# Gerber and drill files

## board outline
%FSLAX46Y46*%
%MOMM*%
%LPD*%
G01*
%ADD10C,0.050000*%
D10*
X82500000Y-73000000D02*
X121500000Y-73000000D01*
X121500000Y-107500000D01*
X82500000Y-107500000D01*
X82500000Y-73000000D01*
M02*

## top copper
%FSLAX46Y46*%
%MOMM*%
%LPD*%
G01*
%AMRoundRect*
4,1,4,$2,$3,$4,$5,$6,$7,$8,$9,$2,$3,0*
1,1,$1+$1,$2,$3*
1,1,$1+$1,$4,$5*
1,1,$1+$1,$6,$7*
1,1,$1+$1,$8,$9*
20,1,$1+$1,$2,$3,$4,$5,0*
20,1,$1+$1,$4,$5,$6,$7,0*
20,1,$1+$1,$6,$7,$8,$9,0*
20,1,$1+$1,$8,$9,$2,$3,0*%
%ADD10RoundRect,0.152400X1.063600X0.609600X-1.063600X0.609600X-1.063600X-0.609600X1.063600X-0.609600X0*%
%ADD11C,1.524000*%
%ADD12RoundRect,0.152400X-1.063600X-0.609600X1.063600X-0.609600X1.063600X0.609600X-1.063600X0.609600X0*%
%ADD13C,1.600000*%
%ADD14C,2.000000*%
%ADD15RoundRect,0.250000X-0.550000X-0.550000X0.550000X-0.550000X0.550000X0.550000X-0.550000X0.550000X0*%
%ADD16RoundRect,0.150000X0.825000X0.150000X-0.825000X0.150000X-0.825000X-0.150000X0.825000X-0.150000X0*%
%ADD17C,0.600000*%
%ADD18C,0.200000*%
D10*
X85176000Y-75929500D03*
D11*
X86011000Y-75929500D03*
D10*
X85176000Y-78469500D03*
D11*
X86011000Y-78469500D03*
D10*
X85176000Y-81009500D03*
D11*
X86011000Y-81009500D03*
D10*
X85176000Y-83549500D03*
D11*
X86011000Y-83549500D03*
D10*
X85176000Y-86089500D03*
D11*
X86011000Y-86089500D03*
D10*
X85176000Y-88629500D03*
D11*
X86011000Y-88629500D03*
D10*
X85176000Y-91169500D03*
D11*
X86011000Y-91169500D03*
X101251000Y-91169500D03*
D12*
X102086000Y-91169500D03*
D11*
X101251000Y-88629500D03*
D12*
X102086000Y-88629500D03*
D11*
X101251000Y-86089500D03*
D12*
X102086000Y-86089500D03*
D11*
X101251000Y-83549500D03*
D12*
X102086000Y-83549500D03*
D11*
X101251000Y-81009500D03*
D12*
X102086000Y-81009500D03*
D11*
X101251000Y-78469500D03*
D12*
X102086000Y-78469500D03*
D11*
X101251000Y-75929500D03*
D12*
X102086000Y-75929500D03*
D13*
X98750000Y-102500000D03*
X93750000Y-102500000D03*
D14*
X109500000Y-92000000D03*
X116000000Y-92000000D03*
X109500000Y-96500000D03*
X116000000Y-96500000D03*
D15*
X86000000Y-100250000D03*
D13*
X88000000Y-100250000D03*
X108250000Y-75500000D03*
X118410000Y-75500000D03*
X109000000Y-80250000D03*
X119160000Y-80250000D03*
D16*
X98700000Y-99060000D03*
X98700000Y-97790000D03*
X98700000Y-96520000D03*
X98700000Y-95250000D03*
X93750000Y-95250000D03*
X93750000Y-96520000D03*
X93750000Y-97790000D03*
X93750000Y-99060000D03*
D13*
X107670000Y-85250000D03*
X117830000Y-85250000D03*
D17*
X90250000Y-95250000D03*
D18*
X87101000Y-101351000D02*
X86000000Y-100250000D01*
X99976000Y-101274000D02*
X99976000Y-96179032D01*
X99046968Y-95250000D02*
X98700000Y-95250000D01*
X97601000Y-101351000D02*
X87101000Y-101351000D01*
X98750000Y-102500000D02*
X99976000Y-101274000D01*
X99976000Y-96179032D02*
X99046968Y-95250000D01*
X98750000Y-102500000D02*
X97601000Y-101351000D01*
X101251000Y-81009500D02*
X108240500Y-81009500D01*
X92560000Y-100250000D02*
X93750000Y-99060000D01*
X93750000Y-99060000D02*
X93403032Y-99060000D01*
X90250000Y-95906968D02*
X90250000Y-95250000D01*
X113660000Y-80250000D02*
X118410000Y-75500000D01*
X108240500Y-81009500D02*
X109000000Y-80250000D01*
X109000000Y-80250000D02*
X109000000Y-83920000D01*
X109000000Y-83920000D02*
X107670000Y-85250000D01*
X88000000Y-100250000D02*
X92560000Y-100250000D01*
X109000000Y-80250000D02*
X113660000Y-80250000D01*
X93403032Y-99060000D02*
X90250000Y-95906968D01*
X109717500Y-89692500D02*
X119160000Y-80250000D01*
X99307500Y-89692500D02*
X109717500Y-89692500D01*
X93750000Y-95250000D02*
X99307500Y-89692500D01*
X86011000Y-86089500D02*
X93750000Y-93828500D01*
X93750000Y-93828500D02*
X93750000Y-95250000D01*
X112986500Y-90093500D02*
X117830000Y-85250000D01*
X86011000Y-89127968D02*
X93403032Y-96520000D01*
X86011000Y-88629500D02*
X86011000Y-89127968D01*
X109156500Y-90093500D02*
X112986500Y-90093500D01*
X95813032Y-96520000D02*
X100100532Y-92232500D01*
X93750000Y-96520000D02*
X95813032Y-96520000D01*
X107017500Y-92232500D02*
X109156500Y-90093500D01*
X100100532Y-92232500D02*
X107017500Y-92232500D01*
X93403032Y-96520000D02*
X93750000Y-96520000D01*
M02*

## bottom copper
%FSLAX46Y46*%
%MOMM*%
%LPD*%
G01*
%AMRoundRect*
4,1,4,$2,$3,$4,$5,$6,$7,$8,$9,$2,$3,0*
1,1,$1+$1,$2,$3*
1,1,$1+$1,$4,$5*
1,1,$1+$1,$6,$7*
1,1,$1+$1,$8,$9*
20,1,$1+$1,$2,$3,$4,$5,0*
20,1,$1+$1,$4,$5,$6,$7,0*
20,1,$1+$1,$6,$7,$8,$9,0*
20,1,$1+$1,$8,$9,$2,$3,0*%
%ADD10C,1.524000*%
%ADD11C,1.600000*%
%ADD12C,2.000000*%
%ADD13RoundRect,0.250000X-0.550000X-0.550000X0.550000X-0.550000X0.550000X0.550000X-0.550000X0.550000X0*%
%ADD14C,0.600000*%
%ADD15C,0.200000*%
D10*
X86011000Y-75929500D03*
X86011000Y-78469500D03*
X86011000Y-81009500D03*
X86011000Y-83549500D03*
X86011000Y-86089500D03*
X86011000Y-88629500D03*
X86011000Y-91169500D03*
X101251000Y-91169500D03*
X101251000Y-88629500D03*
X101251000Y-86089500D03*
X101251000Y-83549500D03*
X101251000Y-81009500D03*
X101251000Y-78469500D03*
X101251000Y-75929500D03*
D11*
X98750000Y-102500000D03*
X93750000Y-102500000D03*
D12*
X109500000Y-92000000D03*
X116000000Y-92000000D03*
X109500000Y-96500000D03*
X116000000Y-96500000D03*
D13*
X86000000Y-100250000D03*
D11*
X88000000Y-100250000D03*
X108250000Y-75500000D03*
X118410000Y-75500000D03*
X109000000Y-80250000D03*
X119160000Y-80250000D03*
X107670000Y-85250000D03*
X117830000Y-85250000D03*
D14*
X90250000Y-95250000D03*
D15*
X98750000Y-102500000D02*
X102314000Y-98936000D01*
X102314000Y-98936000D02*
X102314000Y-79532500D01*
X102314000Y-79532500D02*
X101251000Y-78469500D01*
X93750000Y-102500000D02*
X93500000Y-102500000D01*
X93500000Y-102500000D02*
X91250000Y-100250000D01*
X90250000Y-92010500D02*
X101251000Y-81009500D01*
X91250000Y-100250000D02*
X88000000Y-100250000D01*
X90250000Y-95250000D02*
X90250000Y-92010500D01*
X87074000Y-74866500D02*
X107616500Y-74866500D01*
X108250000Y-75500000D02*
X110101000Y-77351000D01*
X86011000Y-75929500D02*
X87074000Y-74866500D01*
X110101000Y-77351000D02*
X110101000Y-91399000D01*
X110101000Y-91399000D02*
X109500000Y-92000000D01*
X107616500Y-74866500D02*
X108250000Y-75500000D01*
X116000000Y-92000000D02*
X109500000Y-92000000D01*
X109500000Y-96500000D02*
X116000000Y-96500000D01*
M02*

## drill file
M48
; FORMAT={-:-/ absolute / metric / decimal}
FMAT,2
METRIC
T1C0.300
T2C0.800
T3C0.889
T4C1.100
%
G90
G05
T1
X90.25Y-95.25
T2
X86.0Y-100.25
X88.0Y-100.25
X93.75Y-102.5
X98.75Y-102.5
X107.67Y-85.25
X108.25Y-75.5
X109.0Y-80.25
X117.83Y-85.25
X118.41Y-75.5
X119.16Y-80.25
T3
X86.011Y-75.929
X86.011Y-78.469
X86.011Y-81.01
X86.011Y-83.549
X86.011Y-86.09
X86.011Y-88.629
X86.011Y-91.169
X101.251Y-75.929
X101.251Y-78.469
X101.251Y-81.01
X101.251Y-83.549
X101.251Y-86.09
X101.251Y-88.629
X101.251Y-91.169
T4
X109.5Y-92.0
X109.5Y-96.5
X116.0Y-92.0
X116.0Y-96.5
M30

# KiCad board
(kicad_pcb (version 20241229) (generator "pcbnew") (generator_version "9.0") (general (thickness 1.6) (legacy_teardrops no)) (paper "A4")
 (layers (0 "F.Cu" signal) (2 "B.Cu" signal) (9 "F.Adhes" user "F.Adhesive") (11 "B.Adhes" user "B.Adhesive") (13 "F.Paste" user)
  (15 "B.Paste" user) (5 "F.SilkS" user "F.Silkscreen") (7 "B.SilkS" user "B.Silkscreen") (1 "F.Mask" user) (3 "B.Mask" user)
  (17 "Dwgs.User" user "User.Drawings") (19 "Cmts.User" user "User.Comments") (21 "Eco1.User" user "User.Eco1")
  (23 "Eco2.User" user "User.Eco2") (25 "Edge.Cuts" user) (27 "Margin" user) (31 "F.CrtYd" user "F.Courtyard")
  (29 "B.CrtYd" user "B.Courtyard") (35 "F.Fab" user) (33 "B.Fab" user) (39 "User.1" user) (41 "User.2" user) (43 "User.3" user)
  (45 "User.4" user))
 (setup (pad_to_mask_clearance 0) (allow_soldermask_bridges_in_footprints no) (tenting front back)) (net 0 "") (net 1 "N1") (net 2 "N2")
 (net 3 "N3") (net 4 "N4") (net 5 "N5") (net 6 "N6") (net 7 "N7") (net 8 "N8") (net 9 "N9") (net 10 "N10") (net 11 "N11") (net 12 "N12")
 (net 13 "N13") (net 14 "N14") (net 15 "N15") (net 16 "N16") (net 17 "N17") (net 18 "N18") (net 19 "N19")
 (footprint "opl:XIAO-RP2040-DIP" (layer "F.Cu") (at 93.631 83.5495)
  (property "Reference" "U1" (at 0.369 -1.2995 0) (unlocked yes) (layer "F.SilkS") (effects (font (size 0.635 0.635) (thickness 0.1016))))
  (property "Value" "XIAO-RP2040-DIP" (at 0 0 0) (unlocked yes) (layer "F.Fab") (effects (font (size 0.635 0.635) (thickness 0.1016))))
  (pad "1" smd roundrect (at -8.455 -7.62 180) (size 2.432 1.524) (layers "F.Cu" "F.Mask") (roundrect_rratio 0.1) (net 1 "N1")
   (thermal_bridge_angle 45))
  (pad "1" thru_hole circle (at -7.62 -7.62 180) (size 1.524 1.524) (drill 0.889) (layers "*.Cu" "*.Mask") (remove_unused_layers no)
   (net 1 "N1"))
  (pad "2" smd roundrect (at -8.455 -5.08 180) (size 2.432 1.524) (layers "F.Cu" "F.Mask") (roundrect_rratio 0.1) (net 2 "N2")
   (thermal_bridge_angle 45))
  (pad "2" thru_hole circle (at -7.62 -5.08 180) (size 1.524 1.524) (drill 0.889) (layers "*.Cu" "*.Mask") (remove_unused_layers no)
   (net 2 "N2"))
  (pad "3" smd roundrect (at -8.455 -2.54 180) (size 2.432 1.524) (layers "F.Cu" "F.Mask") (roundrect_rratio 0.1) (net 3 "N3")
   (thermal_bridge_angle 45))
  (pad "3" thru_hole circle (at -7.62 -2.54 180) (size 1.524 1.524) (drill 0.889) (layers "*.Cu" "*.Mask") (remove_unused_layers no)
   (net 3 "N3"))
  (pad "4" smd roundrect (at -8.455 0 180) (size 2.432 1.524) (layers "F.Cu" "F.Mask") (roundrect_rratio 0.1) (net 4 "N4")
   (thermal_bridge_angle 45))
  (pad "4" thru_hole circle (at -7.62 0 180) (size 1.524 1.524) (drill 0.889) (layers "*.Cu" "*.Mask") (remove_unused_layers no)
   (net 4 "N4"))
  (pad "5" smd roundrect (at -8.455 2.54 180) (size 2.432 1.524) (layers "F.Cu" "F.Mask") (roundrect_rratio 0.1) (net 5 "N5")
   (thermal_bridge_angle 45))
  (pad "5" thru_hole circle (at -7.62 2.54 180) (size 1.524 1.524) (drill 0.889) (layers "*.Cu" "*.Mask") (remove_unused_layers no)
   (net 5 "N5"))
  (pad "6" smd roundrect (at -8.455 5.08 180) (size 2.432 1.524) (layers "F.Cu" "F.Mask") (roundrect_rratio 0.1) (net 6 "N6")
   (thermal_bridge_angle 45))
  (pad "6" thru_hole circle (at -7.62 5.08 180) (size 1.524 1.524) (drill 0.889) (layers "*.Cu" "*.Mask") (remove_unused_layers no)
   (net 6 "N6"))
  (pad "7" smd roundrect (at -8.455 7.62 180) (size 2.432 1.524) (layers "F.Cu" "F.Mask") (roundrect_rratio 0.1) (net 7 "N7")
   (thermal_bridge_angle 45))
  (pad "7" thru_hole circle (at -7.62 7.62 180) (size 1.524 1.524) (drill 0.889) (layers "*.Cu" "*.Mask") (remove_unused_layers no)
   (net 7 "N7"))
  (pad "8" thru_hole circle (at 7.62 7.62) (size 1.524 1.524) (drill 0.889) (layers "*.Cu" "*.Mask") (remove_unused_layers no) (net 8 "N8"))
  (pad "8" smd roundrect (at 8.455 7.62) (size 2.432 1.524) (layers "F.Cu" "F.Mask") (roundrect_rratio 0.1) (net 8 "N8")
   (thermal_bridge_angle 45))
  (pad "9" thru_hole circle (at 7.62 5.08) (size 1.524 1.524) (drill 0.889) (layers "*.Cu" "*.Mask") (remove_unused_layers no) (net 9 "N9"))
  (pad "9" smd roundrect (at 8.455 5.08) (size 2.432 1.524) (layers "F.Cu" "F.Mask") (roundrect_rratio 0.1) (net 9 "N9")
   (thermal_bridge_angle 45))
  (pad "10" thru_hole circle (at 7.62 2.54) (size 1.524 1.524) (drill 0.889) (layers "*.Cu" "*.Mask") (remove_unused_layers no)
   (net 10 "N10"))
  (pad "10" smd roundrect (at 8.455 2.54) (size 2.432 1.524) (layers "F.Cu" "F.Mask") (roundrect_rratio 0.1) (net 10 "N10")
   (thermal_bridge_angle 45))
  (pad "11" thru_hole circle (at 7.62 0) (size 1.524 1.524) (drill 0.889) (layers "*.Cu" "*.Mask") (remove_unused_layers no) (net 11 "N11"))
  (pad "11" smd roundrect (at 8.455 0) (size 2.432 1.524) (layers "F.Cu" "F.Mask") (roundrect_rratio 0.1) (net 11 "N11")
   (thermal_bridge_angle 45))
  (pad "12" thru_hole circle (at 7.62 -2.54) (size 1.524 1.524) (drill 0.889) (layers "*.Cu" "*.Mask") (remove_unused_layers no)
   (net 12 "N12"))
  (pad "12" smd roundrect (at 8.455 -2.54) (size 2.432 1.524) (layers "F.Cu" "F.Mask") (roundrect_rratio 0.1) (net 12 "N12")
   (thermal_bridge_angle 45))
  (pad "13" thru_hole circle (at 7.62 -5.08) (size 1.524 1.524) (drill 0.889) (layers "*.Cu" "*.Mask") (remove_unused_layers no)
   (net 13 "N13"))
  (pad "13" smd roundrect (at 8.455 -5.08) (size 2.432 1.524) (layers "F.Cu" "F.Mask") (roundrect_rratio 0.1) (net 13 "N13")
   (thermal_bridge_angle 45))
  (pad "14" thru_hole circle (at 7.62 -7.62) (size 1.524 1.524) (drill 0.889) (layers "*.Cu" "*.Mask") (remove_unused_layers no)
   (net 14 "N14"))
  (pad "14" smd roundrect (at 8.455 -7.62) (size 2.432 1.524) (layers "F.Cu" "F.Mask") (roundrect_rratio 0.1) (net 14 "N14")
   (thermal_bridge_angle 45)))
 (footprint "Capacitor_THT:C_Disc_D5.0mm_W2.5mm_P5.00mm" (layer "F.Cu") (at 98.75 102.5 180)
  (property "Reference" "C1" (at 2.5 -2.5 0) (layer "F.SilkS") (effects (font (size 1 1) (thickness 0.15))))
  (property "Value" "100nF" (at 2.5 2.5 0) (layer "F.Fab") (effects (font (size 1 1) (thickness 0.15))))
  (pad "1" thru_hole circle (at 0 0 180) (size 1.6 1.6) (drill 0.8) (layers "*.Cu" "*.Mask") (remove_unused_layers no) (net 13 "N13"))
  (pad "2" thru_hole circle (at 5 0 180) (size 1.6 1.6) (drill 0.8) (layers "*.Cu" "*.Mask") (remove_unused_layers no) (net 12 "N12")))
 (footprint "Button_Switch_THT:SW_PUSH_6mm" (layer "F.Cu") (at 109.5 92)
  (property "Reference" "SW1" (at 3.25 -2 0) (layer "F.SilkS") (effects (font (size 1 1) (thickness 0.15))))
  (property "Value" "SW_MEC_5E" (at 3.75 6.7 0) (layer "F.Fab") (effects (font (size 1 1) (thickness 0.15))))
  (pad "1" thru_hole circle (at 0 0 90) (size 2 2) (drill 1.1) (layers "*.Cu" "*.Mask") (remove_unused_layers no) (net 1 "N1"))
  (pad "1" thru_hole circle (at 6.5 0 90) (size 2 2) (drill 1.1) (layers "*.Cu" "*.Mask") (remove_unused_layers no) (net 1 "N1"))
  (pad "2" thru_hole circle (at 0 4.5 90) (size 2 2) (drill 1.1) (layers "*.Cu" "*.Mask") (remove_unused_layers no) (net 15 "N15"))
  (pad "2" thru_hole circle (at 6.5 4.5 90) (size 2 2) (drill 1.1) (layers "*.Cu" "*.Mask") (remove_unused_layers no) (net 15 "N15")))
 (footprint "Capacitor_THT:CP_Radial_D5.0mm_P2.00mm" (layer "F.Cu") (at 86 100.25)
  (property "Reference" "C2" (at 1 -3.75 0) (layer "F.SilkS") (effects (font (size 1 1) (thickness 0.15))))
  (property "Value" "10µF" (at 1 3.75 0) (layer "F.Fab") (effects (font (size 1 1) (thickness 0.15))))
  (pad "1" thru_hole roundrect (at 0 0) (size 1.6 1.6) (drill 0.8) (layers "*.Cu" "*.Mask") (remove_unused_layers no)
   (roundrect_rratio 0.15625) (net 13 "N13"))
  (pad "2" thru_hole circle (at 2 0) (size 1.6 1.6) (drill 0.8) (layers "*.Cu" "*.Mask") (remove_unused_layers no) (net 12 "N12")))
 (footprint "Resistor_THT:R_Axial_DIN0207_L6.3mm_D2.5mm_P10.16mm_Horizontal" (layer "F.Cu") (at 108.25 75.5)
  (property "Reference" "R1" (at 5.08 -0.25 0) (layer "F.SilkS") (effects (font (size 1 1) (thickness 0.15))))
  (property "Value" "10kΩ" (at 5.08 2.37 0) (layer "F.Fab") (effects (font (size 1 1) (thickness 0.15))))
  (pad "1" thru_hole circle (at 0 0) (size 1.6 1.6) (drill 0.8) (layers "*.Cu" "*.Mask") (remove_unused_layers no) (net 1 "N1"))
  (pad "2" thru_hole circle (at 10.16 0) (size 1.6 1.6) (drill 0.8) (layers "*.Cu" "*.Mask") (remove_unused_layers no) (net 12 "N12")))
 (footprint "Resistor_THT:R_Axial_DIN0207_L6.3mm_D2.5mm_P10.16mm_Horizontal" (layer "F.Cu") (at 109 80.25)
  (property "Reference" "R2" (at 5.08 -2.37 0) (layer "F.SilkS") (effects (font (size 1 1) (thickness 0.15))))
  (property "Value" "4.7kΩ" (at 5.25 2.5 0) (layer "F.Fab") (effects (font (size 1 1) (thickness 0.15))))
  (pad "1" thru_hole circle (at 0 0) (size 1.6 1.6) (drill 0.8) (layers "*.Cu" "*.Mask") (remove_unused_layers no) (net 12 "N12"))
  (pad "2" thru_hole circle (at 10.16 0) (size 1.6 1.6) (drill 0.8) (layers "*.Cu" "*.Mask") (remove_unused_layers no) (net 5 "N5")))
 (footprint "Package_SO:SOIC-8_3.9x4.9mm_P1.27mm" (layer "F.Cu") (at 96.225 97.155 180)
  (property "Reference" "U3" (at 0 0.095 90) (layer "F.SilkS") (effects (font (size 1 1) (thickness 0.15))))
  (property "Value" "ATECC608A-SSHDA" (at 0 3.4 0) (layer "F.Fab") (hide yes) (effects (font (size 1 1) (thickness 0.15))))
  (pad "1" smd roundrect (at -2.475 -1.905 180) (size 1.95 0.6) (layers "F.Cu" "F.Mask" "F.Paste") (roundrect_rratio 0.25) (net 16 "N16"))
  (pad "2" smd roundrect (at -2.475 -0.635 180) (size 1.95 0.6) (layers "F.Cu" "F.Mask" "F.Paste") (roundrect_rratio 0.25) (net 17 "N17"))
  (pad "3" smd roundrect (at -2.475 0.635 180) (size 1.95 0.6) (layers "F.Cu" "F.Mask" "F.Paste") (roundrect_rratio 0.25) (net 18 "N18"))
  (pad "4" smd roundrect (at -2.475 1.905 180) (size 1.95 0.6) (layers "F.Cu" "F.Mask" "F.Paste") (roundrect_rratio 0.25) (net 13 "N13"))
  (pad "5" smd roundrect (at 2.475 1.905 180) (size 1.95 0.6) (layers "F.Cu" "F.Mask" "F.Paste") (roundrect_rratio 0.25) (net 5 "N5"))
  (pad "6" smd roundrect (at 2.475 0.635 180) (size 1.95 0.6) (layers "F.Cu" "F.Mask" "F.Paste") (roundrect_rratio 0.25) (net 6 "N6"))
  (pad "7" smd roundrect (at 2.475 -0.635 180) (size 1.95 0.6) (layers "F.Cu" "F.Mask" "F.Paste") (roundrect_rratio 0.25) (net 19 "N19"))
  (pad "8" smd roundrect (at 2.475 -1.905 180) (size 1.95 0.6) (layers "F.Cu" "F.Mask" "F.Paste") (roundrect_rratio 0.25) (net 12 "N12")))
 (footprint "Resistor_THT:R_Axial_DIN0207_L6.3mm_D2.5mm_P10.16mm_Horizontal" (layer "F.Cu") (at 107.67 85.25)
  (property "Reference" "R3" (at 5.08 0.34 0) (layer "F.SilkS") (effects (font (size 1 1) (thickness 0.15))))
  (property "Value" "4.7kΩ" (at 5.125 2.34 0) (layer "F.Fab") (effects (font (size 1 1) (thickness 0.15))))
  (pad "1" thru_hole circle (at 0 0) (size 1.6 1.6) (drill 0.8) (layers "*.Cu" "*.Mask") (remove_unused_layers no) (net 12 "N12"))
  (pad "2" thru_hole circle (at 10.16 0) (size 1.6 1.6) (drill 0.8) (layers "*.Cu" "*.Mask") (remove_unused_layers no) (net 6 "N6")))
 (gr_rect (start 82.5 73) (end 121.5 107.5) (stroke (width 0.05) (type default)) (fill no) (layer "Edge.Cuts"))
 (segment (start 87.101 101.351) (end 86 100.25) (width 0.2) (layer "F.Cu") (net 13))
 (segment (start 99.976 101.274) (end 99.976 96.179032) (width 0.2) (layer "F.Cu") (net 13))
 (segment (start 99.046968 95.25) (end 98.7 95.25) (width 0.2) (layer "F.Cu") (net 13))
 (segment (start 97.601 101.351) (end 87.101 101.351) (width 0.2) (layer "F.Cu") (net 13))
 (segment (start 98.75 102.5) (end 99.976 101.274) (width 0.2) (layer "F.Cu") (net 13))
 (segment (start 99.976 96.179032) (end 99.046968 95.25) (width 0.2) (layer "F.Cu") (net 13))
 (segment (start 98.75 102.5) (end 97.601 101.351) (width 0.2) (layer "F.Cu") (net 13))
 (segment (start 98.75 102.5) (end 102.314 98.936) (width 0.2) (layer "B.Cu") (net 13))
 (segment (start 102.314 98.936) (end 102.314 79.5325) (width 0.2) (layer "B.Cu") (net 13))
 (segment (start 102.314 79.5325) (end 101.251 78.4695) (width 0.2) (layer "B.Cu") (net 13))
 (segment (start 101.251 81.0095) (end 108.2405 81.0095) (width 0.2) (layer "F.Cu") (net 12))
 (segment (start 92.56 100.25) (end 93.75 99.06) (width 0.2) (layer "F.Cu") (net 12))
 (segment (start 93.75 99.06) (end 93.403032 99.06) (width 0.2) (layer "F.Cu") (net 12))
 (segment (start 90.25 95.906968) (end 90.25 95.25) (width 0.2) (layer "F.Cu") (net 12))
 (segment (start 113.66 80.25) (end 118.41 75.5) (width 0.2) (layer "F.Cu") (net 12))
 (segment (start 108.2405 81.0095) (end 109 80.25) (width 0.2) (layer "F.Cu") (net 12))
 (segment (start 109 80.25) (end 109 83.92) (width 0.2) (layer "F.Cu") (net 12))
 (segment (start 109 83.92) (end 107.67 85.25) (width 0.2) (layer "F.Cu") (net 12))
 (segment (start 88 100.25) (end 92.56 100.25) (width 0.2) (layer "F.Cu") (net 12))
 (segment (start 109 80.25) (end 113.66 80.25) (width 0.2) (layer "F.Cu") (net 12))
 (segment (start 93.403032 99.06) (end 90.25 95.906968) (width 0.2) (layer "F.Cu") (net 12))
 (via (at 90.25 95.25) (size 0.6) (drill 0.3) (layers "F.Cu" "B.Cu") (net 12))
 (segment (start 93.75 102.5) (end 93.5 102.5) (width 0.2) (layer "B.Cu") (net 12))
 (segment (start 93.5 102.5) (end 91.25 100.25) (width 0.2) (layer "B.Cu") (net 12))
 (segment (start 90.25 92.0105) (end 101.251 81.0095) (width 0.2) (layer "B.Cu") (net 12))
 (segment (start 91.25 100.25) (end 88 100.25) (width 0.2) (layer "B.Cu") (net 12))
 (segment (start 90.25 95.25) (end 90.25 92.0105) (width 0.2) (layer "B.Cu") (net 12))
 (segment (start 87.074 74.8665) (end 107.6165 74.8665) (width 0.2) (layer "B.Cu") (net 1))
 (segment (start 108.25 75.5) (end 110.101 77.351) (width 0.2) (layer "B.Cu") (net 1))
 (segment (start 86.011 75.9295) (end 87.074 74.8665) (width 0.2) (layer "B.Cu") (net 1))
 (segment (start 110.101 77.351) (end 110.101 91.399) (width 0.2) (layer "B.Cu") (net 1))
 (segment (start 110.101 91.399) (end 109.5 92) (width 0.2) (layer "B.Cu") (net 1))
 (segment (start 107.6165 74.8665) (end 108.25 75.5) (width 0.2) (layer "B.Cu") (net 1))
 (segment (start 116 92) (end 109.5 92) (width 0.2) (layer "B.Cu") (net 1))
 (segment (start 109.7175 89.6925) (end 119.16 80.25) (width 0.2) (layer "F.Cu") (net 5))
 (segment (start 99.3075 89.6925) (end 109.7175 89.6925) (width 0.2) (layer "F.Cu") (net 5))
 (segment (start 93.75 95.25) (end 99.3075 89.6925) (width 0.2) (layer "F.Cu") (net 5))
 (segment (start 86.011 86.0895) (end 93.75 93.8285) (width 0.2) (layer "F.Cu") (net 5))
 (segment (start 93.75 93.8285) (end 93.75 95.25) (width 0.2) (layer "F.Cu") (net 5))
 (segment (start 112.9865 90.0935) (end 117.83 85.25) (width 0.2) (layer "F.Cu") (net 6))
 (segment (start 86.011 89.127968) (end 93.403032 96.52) (width 0.2) (layer "F.Cu") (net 6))
 (segment (start 86.011 88.6295) (end 86.011 89.127968) (width 0.2) (layer "F.Cu") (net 6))
 (segment (start 109.1565 90.0935) (end 112.9865 90.0935) (width 0.2) (layer "F.Cu") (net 6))
 (segment (start 95.813032 96.52) (end 100.100532 92.2325) (width 0.2) (layer "F.Cu") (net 6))
 (segment (start 93.75 96.52) (end 95.813032 96.52) (width 0.2) (layer "F.Cu") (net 6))
 (segment (start 107.0175 92.2325) (end 109.1565 90.0935) (width 0.2) (layer "F.Cu") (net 6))
 (segment (start 100.100532 92.2325) (end 107.0175 92.2325) (width 0.2) (layer "F.Cu") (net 6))
 (segment (start 93.403032 96.52) (end 93.75 96.52) (width 0.2) (layer "F.Cu") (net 6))
 (segment (start 109.5 96.5) (end 116 96.5) (width 0.2) (layer "B.Cu") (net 15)))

